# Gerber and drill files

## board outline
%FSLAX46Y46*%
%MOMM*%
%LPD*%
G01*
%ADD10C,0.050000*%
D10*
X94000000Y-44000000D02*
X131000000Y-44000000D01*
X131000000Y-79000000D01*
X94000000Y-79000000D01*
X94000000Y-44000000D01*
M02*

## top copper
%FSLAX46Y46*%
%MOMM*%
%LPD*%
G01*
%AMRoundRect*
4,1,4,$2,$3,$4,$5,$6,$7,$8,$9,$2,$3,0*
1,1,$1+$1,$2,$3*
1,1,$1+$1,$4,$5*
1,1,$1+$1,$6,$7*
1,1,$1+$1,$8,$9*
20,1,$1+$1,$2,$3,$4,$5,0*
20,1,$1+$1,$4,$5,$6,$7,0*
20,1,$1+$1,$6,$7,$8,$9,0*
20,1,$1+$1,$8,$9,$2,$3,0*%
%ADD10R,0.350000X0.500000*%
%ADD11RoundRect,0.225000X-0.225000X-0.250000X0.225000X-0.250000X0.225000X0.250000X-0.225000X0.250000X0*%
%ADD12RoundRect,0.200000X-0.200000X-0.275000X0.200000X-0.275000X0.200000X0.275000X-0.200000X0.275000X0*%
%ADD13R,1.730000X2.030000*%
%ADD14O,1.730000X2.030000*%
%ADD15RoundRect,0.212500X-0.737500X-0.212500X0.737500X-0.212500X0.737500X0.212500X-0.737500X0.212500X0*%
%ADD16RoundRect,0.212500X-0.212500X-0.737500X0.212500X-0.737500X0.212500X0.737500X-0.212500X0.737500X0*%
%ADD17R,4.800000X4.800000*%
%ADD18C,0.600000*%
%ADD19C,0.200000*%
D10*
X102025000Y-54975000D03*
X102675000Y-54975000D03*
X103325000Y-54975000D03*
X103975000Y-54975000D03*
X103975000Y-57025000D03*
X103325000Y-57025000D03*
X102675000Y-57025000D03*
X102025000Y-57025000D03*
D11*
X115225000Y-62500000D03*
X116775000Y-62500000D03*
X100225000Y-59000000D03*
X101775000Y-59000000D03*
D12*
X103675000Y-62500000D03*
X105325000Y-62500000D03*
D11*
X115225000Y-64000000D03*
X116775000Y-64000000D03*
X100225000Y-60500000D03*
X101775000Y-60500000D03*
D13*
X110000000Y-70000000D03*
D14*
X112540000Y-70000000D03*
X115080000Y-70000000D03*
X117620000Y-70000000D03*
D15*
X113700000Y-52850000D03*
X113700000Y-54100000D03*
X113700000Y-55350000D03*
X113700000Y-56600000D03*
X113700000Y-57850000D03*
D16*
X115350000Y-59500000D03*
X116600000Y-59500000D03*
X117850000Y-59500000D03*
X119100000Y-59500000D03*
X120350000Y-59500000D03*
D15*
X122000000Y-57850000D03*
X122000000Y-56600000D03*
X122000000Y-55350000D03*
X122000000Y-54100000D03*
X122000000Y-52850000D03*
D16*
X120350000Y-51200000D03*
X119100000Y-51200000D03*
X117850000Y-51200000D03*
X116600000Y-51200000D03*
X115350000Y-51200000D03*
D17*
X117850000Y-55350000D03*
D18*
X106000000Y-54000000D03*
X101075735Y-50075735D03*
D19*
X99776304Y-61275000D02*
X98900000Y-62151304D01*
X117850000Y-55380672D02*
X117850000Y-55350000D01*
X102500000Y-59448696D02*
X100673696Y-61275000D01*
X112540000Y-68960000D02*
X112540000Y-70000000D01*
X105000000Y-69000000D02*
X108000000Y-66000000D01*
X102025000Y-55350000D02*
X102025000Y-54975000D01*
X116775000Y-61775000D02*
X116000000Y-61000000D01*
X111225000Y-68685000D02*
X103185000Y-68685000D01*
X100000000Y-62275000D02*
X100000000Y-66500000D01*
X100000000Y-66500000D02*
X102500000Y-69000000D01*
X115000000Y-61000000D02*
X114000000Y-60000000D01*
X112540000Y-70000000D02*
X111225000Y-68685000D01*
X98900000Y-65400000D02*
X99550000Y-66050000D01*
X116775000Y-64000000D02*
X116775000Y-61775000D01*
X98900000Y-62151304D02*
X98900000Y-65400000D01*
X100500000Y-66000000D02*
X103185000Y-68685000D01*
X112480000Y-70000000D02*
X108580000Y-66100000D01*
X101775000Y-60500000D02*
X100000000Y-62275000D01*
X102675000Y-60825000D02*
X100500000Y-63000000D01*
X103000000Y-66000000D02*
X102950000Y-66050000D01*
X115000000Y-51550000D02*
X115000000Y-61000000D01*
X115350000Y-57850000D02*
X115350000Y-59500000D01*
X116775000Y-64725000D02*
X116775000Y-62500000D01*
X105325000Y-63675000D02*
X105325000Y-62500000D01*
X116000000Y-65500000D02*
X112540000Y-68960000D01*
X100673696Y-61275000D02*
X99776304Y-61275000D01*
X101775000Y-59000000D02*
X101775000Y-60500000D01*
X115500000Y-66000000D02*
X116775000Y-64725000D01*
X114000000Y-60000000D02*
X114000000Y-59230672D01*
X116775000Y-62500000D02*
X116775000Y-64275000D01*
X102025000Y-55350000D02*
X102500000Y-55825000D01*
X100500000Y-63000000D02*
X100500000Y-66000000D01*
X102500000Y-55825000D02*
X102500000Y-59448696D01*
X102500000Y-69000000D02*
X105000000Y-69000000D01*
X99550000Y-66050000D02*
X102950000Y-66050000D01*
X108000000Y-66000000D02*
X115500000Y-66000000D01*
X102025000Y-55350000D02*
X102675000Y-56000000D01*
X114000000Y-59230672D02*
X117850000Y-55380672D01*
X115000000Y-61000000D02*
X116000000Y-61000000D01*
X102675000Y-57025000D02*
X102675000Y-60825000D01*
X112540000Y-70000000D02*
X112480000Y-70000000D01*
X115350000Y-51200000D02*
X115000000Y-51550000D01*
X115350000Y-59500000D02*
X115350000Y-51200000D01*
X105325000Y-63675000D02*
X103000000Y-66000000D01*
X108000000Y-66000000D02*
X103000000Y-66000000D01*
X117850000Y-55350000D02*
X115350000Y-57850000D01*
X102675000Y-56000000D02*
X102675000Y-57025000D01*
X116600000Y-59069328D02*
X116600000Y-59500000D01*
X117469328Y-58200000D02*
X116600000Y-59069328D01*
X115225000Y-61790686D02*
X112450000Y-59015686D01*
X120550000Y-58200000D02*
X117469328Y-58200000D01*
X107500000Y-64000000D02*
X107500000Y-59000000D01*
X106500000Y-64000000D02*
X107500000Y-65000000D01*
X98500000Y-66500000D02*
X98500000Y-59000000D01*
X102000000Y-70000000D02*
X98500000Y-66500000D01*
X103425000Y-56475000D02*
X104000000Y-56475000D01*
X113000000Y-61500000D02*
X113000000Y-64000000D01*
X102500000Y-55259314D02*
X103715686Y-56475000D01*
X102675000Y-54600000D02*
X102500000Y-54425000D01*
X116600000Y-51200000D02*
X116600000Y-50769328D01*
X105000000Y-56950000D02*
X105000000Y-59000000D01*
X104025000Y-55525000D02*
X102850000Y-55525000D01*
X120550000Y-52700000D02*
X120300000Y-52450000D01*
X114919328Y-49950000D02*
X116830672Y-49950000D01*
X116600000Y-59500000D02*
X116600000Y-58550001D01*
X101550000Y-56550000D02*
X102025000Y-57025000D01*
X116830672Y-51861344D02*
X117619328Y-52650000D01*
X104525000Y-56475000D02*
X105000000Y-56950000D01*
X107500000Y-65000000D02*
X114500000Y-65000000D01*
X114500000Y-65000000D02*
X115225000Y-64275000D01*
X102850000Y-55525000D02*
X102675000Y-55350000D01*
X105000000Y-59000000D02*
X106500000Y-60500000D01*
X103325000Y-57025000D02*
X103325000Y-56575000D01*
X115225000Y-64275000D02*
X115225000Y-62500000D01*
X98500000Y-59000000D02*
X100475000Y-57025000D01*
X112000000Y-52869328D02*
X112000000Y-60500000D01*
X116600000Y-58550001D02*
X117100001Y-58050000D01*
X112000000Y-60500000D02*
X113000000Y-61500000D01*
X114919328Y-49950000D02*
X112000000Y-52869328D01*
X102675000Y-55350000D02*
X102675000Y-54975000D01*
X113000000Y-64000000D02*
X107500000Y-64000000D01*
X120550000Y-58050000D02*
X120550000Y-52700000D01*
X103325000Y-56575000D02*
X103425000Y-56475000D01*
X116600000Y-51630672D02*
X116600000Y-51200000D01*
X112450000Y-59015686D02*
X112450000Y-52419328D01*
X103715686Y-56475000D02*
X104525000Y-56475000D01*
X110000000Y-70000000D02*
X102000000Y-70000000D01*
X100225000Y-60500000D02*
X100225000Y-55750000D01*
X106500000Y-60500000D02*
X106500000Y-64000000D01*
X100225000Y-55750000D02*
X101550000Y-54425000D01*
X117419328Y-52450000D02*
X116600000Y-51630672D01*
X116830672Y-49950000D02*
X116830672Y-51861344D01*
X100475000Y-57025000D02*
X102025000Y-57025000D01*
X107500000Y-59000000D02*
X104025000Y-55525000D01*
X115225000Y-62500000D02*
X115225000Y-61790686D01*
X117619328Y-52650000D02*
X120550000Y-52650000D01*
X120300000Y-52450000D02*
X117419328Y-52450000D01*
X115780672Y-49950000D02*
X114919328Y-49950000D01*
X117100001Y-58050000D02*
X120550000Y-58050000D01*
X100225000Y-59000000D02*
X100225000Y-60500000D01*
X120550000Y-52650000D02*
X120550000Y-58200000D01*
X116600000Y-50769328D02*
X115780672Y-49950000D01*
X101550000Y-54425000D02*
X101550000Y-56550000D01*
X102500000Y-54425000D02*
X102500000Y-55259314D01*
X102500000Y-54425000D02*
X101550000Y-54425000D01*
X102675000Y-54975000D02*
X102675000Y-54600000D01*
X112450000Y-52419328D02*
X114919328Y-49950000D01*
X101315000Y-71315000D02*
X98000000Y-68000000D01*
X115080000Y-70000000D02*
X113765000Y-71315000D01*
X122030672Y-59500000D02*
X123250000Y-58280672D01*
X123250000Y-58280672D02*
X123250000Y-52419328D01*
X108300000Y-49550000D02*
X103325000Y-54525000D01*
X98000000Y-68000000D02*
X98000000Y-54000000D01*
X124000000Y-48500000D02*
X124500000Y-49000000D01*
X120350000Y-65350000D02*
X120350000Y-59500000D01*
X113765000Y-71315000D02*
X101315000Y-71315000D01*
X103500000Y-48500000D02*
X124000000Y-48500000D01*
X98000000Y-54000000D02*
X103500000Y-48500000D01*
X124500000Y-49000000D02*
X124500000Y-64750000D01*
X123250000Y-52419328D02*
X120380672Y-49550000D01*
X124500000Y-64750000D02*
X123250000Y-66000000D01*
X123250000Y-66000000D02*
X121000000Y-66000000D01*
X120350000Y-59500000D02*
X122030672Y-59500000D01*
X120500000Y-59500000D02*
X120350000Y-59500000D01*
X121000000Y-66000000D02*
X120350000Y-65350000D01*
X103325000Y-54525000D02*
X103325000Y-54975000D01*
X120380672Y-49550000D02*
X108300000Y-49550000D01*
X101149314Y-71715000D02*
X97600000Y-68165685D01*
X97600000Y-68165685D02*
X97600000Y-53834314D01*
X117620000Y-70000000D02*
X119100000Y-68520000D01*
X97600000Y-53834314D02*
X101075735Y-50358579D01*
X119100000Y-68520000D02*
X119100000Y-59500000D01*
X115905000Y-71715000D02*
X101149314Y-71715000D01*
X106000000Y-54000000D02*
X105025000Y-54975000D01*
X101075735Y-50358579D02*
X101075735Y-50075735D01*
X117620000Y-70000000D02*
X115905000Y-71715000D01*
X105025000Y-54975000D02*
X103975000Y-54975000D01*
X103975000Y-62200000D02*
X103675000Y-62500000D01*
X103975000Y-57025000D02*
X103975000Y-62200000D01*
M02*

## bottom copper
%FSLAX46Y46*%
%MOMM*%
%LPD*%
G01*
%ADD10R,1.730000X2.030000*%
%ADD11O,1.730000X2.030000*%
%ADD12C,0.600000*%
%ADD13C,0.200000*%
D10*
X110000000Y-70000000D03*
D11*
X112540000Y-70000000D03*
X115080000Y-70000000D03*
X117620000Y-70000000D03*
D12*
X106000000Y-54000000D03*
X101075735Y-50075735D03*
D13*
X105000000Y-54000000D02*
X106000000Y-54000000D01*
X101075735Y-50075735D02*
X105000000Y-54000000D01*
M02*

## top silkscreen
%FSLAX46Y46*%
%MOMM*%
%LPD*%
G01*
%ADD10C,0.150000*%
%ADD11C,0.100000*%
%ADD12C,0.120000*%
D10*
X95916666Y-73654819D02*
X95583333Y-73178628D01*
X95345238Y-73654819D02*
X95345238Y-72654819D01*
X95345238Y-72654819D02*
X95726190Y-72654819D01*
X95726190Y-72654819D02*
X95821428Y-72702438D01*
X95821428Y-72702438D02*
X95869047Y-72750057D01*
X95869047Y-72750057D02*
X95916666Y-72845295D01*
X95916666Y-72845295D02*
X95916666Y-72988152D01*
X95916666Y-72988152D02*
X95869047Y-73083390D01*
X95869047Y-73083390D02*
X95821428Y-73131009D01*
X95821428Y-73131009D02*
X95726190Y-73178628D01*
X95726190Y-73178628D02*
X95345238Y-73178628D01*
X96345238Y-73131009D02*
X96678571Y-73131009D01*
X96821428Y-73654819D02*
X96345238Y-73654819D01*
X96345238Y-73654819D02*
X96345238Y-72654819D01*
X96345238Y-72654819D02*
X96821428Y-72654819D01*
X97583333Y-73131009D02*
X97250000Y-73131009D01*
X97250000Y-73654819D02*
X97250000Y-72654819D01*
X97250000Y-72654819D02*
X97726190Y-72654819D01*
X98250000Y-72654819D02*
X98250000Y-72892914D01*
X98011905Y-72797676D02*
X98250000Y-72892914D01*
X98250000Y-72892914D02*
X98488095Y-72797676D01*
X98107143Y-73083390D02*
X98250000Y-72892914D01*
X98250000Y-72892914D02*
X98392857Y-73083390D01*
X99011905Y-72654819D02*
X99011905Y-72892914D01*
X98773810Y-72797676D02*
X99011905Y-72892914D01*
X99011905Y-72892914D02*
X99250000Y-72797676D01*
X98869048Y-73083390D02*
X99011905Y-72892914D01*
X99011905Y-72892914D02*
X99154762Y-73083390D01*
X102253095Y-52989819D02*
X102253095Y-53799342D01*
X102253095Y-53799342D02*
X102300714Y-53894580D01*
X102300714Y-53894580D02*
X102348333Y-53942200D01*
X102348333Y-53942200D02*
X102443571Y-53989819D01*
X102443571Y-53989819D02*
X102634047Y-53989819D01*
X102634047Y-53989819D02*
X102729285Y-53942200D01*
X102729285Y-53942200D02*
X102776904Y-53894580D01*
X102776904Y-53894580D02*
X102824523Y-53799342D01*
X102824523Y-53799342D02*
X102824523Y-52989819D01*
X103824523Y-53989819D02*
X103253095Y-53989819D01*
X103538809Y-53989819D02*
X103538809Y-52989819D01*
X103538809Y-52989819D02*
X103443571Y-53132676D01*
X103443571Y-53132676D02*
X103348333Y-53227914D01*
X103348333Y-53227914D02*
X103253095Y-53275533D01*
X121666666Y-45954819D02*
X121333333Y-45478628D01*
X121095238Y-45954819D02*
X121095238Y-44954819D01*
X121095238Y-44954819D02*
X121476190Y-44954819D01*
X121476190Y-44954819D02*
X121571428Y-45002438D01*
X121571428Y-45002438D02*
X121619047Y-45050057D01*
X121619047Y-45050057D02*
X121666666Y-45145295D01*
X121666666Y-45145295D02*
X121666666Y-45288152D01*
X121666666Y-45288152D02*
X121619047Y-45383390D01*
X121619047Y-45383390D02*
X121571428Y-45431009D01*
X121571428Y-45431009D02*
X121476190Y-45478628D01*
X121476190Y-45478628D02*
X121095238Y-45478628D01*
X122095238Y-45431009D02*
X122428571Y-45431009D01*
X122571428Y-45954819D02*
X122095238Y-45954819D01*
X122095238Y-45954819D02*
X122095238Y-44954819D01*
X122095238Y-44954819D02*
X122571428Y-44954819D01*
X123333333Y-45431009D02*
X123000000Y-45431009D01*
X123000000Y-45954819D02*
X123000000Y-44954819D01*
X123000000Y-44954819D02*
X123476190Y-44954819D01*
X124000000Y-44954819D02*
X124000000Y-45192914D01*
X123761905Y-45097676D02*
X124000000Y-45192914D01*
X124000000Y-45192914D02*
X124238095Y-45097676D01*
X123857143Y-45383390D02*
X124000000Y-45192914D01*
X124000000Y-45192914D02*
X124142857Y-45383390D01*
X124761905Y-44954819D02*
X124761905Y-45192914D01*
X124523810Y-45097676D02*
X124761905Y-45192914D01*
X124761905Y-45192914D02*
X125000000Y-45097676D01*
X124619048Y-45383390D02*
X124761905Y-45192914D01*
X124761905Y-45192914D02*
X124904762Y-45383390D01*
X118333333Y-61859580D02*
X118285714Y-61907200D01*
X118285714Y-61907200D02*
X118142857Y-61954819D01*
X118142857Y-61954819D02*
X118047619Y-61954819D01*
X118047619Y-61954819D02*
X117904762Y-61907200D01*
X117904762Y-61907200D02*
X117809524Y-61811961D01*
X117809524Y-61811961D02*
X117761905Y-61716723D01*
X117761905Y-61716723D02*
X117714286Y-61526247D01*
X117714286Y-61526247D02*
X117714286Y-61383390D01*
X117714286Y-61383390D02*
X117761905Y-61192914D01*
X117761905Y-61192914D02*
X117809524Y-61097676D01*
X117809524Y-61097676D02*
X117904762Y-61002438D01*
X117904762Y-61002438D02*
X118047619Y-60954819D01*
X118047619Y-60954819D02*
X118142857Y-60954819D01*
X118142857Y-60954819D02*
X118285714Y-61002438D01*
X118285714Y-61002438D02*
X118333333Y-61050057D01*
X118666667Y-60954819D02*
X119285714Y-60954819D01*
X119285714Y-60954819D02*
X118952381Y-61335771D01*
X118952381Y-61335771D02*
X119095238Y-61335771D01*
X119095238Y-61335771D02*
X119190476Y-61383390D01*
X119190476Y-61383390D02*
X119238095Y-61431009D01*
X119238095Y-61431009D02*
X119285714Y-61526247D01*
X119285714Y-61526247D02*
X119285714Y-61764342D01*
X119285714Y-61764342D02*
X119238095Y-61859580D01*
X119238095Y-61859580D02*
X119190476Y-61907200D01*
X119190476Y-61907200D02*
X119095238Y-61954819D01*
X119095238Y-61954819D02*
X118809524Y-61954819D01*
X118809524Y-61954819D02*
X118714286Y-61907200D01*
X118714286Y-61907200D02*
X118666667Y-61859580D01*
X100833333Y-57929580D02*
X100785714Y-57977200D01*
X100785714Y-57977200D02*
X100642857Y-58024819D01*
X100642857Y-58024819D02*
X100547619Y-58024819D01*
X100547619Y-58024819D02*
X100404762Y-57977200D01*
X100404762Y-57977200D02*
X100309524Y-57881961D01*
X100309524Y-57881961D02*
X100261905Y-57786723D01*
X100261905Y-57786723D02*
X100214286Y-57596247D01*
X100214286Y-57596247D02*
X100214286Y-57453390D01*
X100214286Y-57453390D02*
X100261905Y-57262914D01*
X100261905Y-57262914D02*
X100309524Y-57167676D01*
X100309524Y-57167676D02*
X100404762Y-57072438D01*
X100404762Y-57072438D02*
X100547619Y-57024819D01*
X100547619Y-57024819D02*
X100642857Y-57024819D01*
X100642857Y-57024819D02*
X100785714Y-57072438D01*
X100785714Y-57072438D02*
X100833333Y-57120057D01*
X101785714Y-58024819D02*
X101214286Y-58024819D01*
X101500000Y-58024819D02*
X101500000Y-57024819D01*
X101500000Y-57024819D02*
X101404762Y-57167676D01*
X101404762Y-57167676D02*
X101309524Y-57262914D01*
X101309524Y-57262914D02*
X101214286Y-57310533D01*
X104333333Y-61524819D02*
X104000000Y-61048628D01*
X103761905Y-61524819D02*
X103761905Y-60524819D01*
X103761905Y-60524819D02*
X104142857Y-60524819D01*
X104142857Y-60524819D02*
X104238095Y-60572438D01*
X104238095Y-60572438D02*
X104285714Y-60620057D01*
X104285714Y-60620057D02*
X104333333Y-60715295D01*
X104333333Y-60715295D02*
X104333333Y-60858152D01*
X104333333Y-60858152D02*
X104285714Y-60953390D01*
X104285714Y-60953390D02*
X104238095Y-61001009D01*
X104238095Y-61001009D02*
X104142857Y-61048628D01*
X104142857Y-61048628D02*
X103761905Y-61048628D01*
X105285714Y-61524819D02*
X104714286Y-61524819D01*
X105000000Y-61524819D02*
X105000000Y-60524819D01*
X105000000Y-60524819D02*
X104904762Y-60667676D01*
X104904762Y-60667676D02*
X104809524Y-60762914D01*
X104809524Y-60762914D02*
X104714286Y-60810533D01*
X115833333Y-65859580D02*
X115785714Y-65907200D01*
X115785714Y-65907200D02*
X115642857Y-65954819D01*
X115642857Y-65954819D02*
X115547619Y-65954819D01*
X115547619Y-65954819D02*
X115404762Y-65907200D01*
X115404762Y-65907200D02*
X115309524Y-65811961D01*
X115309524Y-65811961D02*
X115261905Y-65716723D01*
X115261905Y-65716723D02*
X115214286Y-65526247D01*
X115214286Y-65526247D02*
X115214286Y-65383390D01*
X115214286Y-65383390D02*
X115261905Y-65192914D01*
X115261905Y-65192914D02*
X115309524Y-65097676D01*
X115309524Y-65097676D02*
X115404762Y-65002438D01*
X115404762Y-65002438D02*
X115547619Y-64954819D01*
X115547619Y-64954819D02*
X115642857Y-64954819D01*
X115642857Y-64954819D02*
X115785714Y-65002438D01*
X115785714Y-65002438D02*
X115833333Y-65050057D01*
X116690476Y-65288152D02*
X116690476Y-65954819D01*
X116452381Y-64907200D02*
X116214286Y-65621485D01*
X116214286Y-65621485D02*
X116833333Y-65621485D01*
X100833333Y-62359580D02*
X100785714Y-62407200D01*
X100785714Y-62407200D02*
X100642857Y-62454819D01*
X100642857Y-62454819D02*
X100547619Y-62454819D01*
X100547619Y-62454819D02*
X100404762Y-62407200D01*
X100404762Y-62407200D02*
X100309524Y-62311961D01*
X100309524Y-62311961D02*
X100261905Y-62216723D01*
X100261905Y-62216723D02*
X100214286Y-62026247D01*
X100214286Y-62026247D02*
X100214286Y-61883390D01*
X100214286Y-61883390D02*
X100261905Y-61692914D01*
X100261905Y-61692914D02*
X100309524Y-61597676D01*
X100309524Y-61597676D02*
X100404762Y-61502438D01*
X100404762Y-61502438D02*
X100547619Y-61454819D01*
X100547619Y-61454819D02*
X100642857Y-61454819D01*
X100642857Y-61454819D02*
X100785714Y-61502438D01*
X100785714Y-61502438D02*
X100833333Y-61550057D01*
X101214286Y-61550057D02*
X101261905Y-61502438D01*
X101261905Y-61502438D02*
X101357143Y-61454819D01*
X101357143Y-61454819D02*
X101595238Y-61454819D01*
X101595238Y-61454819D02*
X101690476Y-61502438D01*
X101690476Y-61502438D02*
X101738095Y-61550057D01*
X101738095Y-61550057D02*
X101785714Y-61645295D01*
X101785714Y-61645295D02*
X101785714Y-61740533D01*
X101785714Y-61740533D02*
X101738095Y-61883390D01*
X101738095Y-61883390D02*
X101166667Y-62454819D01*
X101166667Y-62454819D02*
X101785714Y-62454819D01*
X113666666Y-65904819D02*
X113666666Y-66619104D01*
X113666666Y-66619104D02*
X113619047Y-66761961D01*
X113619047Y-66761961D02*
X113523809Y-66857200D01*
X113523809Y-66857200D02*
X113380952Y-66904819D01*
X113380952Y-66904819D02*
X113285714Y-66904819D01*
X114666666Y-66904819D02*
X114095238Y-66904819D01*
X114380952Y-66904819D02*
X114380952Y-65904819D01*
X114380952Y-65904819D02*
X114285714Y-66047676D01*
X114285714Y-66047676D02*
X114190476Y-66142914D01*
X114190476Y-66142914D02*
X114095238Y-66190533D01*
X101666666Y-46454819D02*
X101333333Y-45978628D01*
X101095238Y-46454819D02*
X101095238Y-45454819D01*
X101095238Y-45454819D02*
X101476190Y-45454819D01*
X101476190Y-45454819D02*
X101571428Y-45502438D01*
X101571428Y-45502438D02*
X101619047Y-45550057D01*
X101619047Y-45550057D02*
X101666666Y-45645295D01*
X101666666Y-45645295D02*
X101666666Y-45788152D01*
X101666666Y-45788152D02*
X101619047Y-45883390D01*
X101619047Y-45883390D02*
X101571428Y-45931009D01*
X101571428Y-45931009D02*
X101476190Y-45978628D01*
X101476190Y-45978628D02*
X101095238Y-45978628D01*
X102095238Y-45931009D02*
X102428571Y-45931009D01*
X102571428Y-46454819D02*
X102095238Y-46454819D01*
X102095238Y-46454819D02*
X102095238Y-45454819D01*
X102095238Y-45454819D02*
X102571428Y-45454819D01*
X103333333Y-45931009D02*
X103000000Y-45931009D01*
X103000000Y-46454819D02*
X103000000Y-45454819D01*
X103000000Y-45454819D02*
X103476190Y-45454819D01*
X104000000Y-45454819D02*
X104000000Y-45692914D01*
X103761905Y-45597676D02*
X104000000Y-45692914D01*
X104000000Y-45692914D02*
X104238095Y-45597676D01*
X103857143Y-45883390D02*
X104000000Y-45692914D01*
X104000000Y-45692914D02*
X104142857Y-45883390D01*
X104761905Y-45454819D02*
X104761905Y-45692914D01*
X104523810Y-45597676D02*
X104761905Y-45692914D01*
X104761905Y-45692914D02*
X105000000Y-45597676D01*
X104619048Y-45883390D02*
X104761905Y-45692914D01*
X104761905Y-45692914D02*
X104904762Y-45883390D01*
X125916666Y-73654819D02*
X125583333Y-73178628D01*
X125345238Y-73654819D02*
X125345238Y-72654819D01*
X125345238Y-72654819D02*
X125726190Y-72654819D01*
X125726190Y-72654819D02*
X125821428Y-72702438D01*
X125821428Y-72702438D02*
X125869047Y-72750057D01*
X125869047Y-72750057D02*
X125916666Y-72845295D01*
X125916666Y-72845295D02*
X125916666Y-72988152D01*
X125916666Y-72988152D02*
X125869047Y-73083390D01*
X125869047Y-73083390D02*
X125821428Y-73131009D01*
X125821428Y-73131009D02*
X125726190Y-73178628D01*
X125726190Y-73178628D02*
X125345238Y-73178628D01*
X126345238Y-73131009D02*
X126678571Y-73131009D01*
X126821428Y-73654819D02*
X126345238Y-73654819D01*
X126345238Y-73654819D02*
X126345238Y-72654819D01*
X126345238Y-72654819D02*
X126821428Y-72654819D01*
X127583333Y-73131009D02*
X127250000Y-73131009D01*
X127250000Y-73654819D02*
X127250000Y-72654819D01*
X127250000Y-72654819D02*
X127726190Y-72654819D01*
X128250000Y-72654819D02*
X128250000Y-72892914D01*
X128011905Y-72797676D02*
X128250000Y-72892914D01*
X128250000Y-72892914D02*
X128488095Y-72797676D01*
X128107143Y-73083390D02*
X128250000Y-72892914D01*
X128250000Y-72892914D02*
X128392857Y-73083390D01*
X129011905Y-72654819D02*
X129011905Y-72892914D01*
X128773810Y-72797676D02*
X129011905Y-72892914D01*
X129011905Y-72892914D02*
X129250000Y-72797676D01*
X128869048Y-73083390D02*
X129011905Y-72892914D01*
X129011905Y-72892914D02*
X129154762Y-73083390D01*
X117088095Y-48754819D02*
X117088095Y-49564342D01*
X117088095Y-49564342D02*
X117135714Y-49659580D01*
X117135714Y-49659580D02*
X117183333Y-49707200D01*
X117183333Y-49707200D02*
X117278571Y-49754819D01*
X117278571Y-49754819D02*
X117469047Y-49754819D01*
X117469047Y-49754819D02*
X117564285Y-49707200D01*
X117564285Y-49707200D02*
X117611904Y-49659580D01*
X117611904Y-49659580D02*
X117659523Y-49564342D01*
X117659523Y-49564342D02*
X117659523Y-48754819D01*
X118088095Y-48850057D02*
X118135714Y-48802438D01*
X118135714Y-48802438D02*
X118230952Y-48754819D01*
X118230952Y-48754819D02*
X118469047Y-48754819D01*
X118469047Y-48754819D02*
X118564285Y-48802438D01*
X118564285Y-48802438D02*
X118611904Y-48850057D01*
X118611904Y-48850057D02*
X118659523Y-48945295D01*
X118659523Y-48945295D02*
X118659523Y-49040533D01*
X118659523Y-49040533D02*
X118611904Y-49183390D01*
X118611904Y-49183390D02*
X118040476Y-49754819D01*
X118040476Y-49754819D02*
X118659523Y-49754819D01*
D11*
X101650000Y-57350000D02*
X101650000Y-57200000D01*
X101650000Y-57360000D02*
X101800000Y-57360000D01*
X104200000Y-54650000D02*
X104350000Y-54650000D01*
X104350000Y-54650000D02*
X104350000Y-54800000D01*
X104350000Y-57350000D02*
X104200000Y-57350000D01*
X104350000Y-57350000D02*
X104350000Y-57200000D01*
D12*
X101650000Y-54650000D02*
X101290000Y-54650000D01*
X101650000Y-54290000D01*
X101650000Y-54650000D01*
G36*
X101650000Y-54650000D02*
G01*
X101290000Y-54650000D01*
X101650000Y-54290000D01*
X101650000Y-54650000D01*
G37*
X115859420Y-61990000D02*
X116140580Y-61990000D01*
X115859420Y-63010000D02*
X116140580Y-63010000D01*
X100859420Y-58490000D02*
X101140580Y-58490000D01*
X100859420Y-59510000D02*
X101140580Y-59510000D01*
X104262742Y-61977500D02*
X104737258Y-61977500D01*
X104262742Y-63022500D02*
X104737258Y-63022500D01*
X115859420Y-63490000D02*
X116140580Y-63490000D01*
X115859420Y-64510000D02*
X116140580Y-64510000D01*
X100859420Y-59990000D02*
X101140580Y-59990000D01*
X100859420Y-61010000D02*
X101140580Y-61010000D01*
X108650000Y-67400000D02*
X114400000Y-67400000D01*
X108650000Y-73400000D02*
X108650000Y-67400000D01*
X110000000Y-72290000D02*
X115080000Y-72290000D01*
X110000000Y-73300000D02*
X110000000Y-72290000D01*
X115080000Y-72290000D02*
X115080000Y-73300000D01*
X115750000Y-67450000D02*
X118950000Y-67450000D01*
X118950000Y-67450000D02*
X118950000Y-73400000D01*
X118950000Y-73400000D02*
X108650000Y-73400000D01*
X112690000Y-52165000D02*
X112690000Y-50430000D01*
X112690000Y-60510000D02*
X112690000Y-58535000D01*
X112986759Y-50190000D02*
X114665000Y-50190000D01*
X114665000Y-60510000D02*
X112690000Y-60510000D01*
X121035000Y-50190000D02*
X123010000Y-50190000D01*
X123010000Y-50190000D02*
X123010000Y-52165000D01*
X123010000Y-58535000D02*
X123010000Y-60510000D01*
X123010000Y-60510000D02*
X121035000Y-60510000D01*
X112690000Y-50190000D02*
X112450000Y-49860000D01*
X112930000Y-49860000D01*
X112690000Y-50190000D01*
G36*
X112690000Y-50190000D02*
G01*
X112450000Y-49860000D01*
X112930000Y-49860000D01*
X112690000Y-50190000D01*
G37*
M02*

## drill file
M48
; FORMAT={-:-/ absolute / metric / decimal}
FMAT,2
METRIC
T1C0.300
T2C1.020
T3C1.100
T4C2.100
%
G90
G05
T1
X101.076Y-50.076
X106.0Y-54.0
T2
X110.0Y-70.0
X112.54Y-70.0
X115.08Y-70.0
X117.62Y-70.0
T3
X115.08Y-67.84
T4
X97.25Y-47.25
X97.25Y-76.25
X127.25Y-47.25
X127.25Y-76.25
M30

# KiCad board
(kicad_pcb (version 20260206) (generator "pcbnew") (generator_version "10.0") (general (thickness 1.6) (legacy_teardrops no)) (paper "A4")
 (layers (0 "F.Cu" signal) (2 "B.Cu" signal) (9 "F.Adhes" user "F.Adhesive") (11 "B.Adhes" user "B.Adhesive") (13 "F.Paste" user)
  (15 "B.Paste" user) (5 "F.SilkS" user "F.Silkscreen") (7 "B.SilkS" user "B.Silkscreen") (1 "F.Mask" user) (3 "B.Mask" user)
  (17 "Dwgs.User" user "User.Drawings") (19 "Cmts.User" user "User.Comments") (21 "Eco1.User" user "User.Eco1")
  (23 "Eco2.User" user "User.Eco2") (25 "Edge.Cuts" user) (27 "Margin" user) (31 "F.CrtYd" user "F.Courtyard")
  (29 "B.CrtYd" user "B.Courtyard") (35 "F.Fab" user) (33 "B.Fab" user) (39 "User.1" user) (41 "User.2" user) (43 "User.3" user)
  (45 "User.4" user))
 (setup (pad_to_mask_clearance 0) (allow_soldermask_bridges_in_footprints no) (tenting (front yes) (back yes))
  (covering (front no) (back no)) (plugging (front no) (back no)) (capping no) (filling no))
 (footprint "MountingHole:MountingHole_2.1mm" (layer "F.Cu") (at 97.25 76.25)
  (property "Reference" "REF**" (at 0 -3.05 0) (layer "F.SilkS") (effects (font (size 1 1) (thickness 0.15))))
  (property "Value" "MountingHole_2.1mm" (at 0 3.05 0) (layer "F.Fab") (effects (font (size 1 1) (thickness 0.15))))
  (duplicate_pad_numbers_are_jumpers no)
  (pad "" np_thru_hole circle (at 0 0) (size 2.1 2.1) (drill 2.1) (layers "*.Cu" "*.Mask")))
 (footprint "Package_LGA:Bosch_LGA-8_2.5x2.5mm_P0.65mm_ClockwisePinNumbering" (layer "F.Cu") (at 103 56)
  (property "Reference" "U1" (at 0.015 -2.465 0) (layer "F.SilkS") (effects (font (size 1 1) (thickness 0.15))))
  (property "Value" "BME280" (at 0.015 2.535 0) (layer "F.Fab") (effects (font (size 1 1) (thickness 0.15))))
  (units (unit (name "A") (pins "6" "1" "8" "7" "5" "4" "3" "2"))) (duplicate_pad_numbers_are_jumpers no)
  (fp_line (start -1.35 1.35) (end -1.35 1.2) (stroke (width 0.1) (type solid)) (layer "F.SilkS"))
  (fp_line (start -1.35 1.36) (end -1.2 1.36) (stroke (width 0.1) (type solid)) (layer "F.SilkS"))
  (fp_line (start 1.2 -1.35) (end 1.35 -1.35) (stroke (width 0.1) (type solid)) (layer "F.SilkS"))
  (fp_line (start 1.35 -1.35) (end 1.35 -1.2) (stroke (width 0.1) (type solid)) (layer "F.SilkS"))
  (fp_line (start 1.35 1.35) (end 1.2 1.35) (stroke (width 0.1) (type solid)) (layer "F.SilkS"))
  (fp_line (start 1.35 1.35) (end 1.35 1.2) (stroke (width 0.1) (type solid)) (layer "F.SilkS"))
  (fp_poly
   (pts (xy -1.35 -1.35) (xy -1.71 -1.35) (xy -1.35 -1.71) (xy -1.35 -1.35)) (stroke (width 0.12) (type solid)) (fill yes) (layer "F.SilkS"))
  (pad "1" smd rect (at -0.975 -1.025 90) (size 0.5 0.35) (layers "F.Cu" "F.Mask" "F.Paste") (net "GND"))
  (pad "2" smd rect (at -0.325 -1.025 90) (size 0.5 0.35) (layers "F.Cu" "F.Mask" "F.Paste") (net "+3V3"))
  (pad "3" smd rect (at 0.325 -1.025 90) (size 0.5 0.35) (layers "F.Cu" "F.Mask" "F.Paste") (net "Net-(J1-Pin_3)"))
  (pad "4" smd rect (at 0.975 -1.025 90) (size 0.5 0.35) (layers "F.Cu" "F.Mask" "F.Paste") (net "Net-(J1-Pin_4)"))
  (pad "5" smd rect (at 0.975 1.025 90) (size 0.5 0.35) (layers "F.Cu" "F.Mask" "F.Paste") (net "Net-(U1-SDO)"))
  (pad "6" smd rect (at 0.325 1.025 90) (size 0.5 0.35) (layers "F.Cu" "F.Mask" "F.Paste") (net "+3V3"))
  (pad "7" smd rect (at -0.325 1.025 90) (size 0.5 0.35) (layers "F.Cu" "F.Mask" "F.Paste") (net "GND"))
  (pad "8" smd rect (at -0.975 1.025 90) (size 0.5 0.35) (layers "F.Cu" "F.Mask" "F.Paste") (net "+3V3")))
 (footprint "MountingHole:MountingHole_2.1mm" (layer "F.Cu") (at 127.25 47.25)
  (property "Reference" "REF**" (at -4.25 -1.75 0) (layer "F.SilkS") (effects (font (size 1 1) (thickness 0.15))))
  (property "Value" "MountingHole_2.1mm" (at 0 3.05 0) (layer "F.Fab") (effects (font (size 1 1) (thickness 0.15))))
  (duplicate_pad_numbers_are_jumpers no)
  (pad "" np_thru_hole circle (at 0 0) (size 2.1 2.1) (drill 2.1) (layers "*.Cu" "*.Mask")))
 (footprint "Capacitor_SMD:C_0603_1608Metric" (layer "F.Cu") (at 116 62.5)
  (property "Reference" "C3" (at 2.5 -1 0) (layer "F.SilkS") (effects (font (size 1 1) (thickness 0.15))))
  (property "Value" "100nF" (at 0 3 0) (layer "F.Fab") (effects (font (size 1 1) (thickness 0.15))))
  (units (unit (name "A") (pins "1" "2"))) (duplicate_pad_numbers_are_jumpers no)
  (fp_line (start -0.14058 -0.51) (end 0.14058 -0.51) (stroke (width 0.12) (type solid)) (layer "F.SilkS"))
  (fp_line (start -0.14058 0.51) (end 0.14058 0.51) (stroke (width 0.12) (type solid)) (layer "F.SilkS"))
  (pad "1" smd roundrect (at -0.775 0) (size 0.9 0.95) (layers "F.Cu" "F.Mask" "F.Paste") (roundrect_rratio 0.25) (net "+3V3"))
  (pad "2" smd roundrect (at 0.775 0) (size 0.9 0.95) (layers "F.Cu" "F.Mask" "F.Paste") (roundrect_rratio 0.25) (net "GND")))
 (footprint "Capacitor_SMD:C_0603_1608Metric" (layer "F.Cu") (at 101 59)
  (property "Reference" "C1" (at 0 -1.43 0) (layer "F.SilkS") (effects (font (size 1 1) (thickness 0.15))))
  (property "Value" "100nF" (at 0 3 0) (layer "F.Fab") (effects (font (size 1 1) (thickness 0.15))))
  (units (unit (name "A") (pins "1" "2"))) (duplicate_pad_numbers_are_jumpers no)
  (fp_line (start -0.14058 -0.51) (end 0.14058 -0.51) (stroke (width 0.12) (type solid)) (layer "F.SilkS"))
  (fp_line (start -0.14058 0.51) (end 0.14058 0.51) (stroke (width 0.12) (type solid)) (layer "F.SilkS"))
  (pad "1" smd roundrect (at -0.775 0) (size 0.9 0.95) (layers "F.Cu" "F.Mask" "F.Paste") (roundrect_rratio 0.25) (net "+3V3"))
  (pad "2" smd roundrect (at 0.775 0) (size 0.9 0.95) (layers "F.Cu" "F.Mask" "F.Paste") (roundrect_rratio 0.25) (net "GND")))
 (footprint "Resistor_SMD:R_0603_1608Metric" (layer "F.Cu") (at 104.5 62.5)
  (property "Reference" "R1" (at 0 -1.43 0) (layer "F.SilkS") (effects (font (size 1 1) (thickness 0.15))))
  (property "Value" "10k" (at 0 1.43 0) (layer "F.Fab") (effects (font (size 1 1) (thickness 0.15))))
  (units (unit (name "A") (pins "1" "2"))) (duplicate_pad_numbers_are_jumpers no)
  (fp_line (start -0.237258 -0.5225) (end 0.237258 -0.5225) (stroke (width 0.12) (type solid)) (layer "F.SilkS"))
  (fp_line (start -0.237258 0.5225) (end 0.237258 0.5225) (stroke (width 0.12) (type solid)) (layer "F.SilkS"))
  (pad "1" smd roundrect (at -0.825 0) (size 0.8 0.95) (layers "F.Cu" "F.Mask" "F.Paste") (roundrect_rratio 0.25) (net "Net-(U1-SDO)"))
  (pad "2" smd roundrect (at 0.825 0) (size 0.8 0.95) (layers "F.Cu" "F.Mask" "F.Paste") (roundrect_rratio 0.25) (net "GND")))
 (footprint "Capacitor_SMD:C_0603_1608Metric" (layer "F.Cu") (at 116 64)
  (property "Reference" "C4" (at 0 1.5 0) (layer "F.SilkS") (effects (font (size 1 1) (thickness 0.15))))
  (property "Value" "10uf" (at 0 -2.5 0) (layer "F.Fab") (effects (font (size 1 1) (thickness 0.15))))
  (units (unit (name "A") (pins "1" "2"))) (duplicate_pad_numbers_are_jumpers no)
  (fp_line (start -0.14058 -0.51) (end 0.14058 -0.51) (stroke (width 0.12) (type solid)) (layer "F.SilkS"))
  (fp_line (start -0.14058 0.51) (end 0.14058 0.51) (stroke (width 0.12) (type solid)) (layer "F.SilkS"))
  (pad "1" smd roundrect (at -0.775 0) (size 0.9 0.95) (layers "F.Cu" "F.Mask" "F.Paste") (roundrect_rratio 0.25) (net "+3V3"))
  (pad "2" smd roundrect (at 0.775 0) (size 0.9 0.95) (layers "F.Cu" "F.Mask" "F.Paste") (roundrect_rratio 0.25) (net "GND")))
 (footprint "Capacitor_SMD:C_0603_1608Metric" (layer "F.Cu") (at 101 60.5)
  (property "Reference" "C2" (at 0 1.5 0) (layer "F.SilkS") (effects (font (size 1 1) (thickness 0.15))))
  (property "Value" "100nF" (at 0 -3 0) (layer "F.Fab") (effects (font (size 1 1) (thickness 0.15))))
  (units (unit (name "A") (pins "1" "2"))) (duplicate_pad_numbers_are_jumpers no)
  (fp_line (start -0.14058 -0.51) (end 0.14058 -0.51) (stroke (width 0.12) (type solid)) (layer "F.SilkS"))
  (fp_line (start -0.14058 0.51) (end 0.14058 0.51) (stroke (width 0.12) (type solid)) (layer "F.SilkS"))
  (pad "1" smd roundrect (at -0.775 0) (size 0.9 0.95) (layers "F.Cu" "F.Mask" "F.Paste") (roundrect_rratio 0.25) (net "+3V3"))
  (pad "2" smd roundrect (at 0.775 0) (size 0.9 0.95) (layers "F.Cu" "F.Mask" "F.Paste") (roundrect_rratio 0.25) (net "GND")))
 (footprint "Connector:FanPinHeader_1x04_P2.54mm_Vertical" (layer "F.Cu") (at 110 70)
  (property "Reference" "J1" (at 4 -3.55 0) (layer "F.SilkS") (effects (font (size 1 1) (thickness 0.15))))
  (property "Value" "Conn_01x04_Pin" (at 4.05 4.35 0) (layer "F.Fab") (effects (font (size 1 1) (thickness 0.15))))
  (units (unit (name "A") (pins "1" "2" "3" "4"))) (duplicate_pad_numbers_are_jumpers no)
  (fp_line (start -1.35 -2.6) (end 4.4 -2.6) (stroke (width 0.12) (type solid)) (layer "F.SilkS"))
  (fp_line (start -1.35 3.4) (end -1.35 -2.6) (stroke (width 0.12) (type solid)) (layer "F.SilkS"))
  (fp_line (start 0 2.29) (end 5.08 2.29) (stroke (width 0.12) (type solid)) (layer "F.SilkS"))
  (fp_line (start 0 3.3) (end 0 2.29) (stroke (width 0.12) (type solid)) (layer "F.SilkS"))
  (fp_line (start 5.08 2.29) (end 5.08 3.3) (stroke (width 0.12) (type solid)) (layer "F.SilkS"))
  (fp_line (start 5.75 -2.55) (end 8.95 -2.55) (stroke (width 0.12) (type solid)) (layer "F.SilkS"))
  (fp_line (start 8.95 -2.55) (end 8.95 3.4) (stroke (width 0.12) (type solid)) (layer "F.SilkS"))
  (fp_line (start 8.95 3.4) (end -1.35 3.4) (stroke (width 0.12) (type solid)) (layer "F.SilkS"))
  (pad "" np_thru_hole circle (at 5.08 -2.16 90) (size 1.1 1.1) (drill 1.1) (layers "*.Cu" "*.Mask"))
  (pad "1" thru_hole rect (at 0 0 90) (size 2.03 1.73) (drill 1.02) (layers "*.Cu" "*.Mask") (remove_unused_layers no) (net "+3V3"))
  (pad "2" thru_hole oval (at 2.54 0 90) (size 2.03 1.73) (drill 1.02) (layers "*.Cu" "*.Mask") (remove_unused_layers no) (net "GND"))
  (pad "3" thru_hole oval (at 5.08 0 90) (size 2.03 1.73) (drill 1.02) (layers "*.Cu" "*.Mask") (remove_unused_layers no)
   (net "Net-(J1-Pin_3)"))
  (pad "4" thru_hole oval (at 7.62 0 90) (size 2.03 1.73) (drill 1.02) (layers "*.Cu" "*.Mask") (remove_unused_layers no)
   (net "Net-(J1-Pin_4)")))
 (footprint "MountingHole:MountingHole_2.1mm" (layer "F.Cu") (at 97.25 47.25)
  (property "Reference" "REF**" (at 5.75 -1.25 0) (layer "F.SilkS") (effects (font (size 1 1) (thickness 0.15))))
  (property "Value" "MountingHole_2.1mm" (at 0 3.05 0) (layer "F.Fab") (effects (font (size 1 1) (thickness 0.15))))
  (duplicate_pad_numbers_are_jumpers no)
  (pad "" np_thru_hole circle (at 0 0) (size 2.1 2.1) (drill 2.1) (layers "*.Cu" "*.Mask")))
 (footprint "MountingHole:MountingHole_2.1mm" (layer "F.Cu") (at 127.25 76.25)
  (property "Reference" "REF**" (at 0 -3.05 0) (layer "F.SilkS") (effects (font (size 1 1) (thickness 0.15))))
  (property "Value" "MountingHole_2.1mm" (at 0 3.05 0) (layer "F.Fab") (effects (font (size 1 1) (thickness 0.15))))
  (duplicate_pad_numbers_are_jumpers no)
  (pad "" np_thru_hole circle (at 0 0) (size 2.1 2.1) (drill 2.1) (layers "*.Cu" "*.Mask")))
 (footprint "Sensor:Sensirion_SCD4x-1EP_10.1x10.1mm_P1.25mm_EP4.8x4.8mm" (layer "F.Cu") (at 117.85 55.35)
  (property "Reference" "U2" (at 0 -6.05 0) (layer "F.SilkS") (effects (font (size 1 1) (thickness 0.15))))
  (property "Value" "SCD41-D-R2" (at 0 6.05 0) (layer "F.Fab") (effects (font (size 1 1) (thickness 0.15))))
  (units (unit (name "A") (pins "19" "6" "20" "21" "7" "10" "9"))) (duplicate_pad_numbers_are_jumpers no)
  (fp_line (start -5.16 -3.185) (end -5.16 -4.92) (stroke (width 0.12) (type solid)) (layer "F.SilkS"))
  (fp_line (start -5.16 5.16) (end -5.16 3.185) (stroke (width 0.12) (type solid)) (layer "F.SilkS"))
  (fp_line (start -4.863241 -5.16) (end -3.185 -5.16) (stroke (width 0.12) (type solid)) (layer "F.SilkS"))
  (fp_line (start -3.185 5.16) (end -5.16 5.16) (stroke (width 0.12) (type solid)) (layer "F.SilkS"))
  (fp_line (start 3.185 -5.16) (end 5.16 -5.16) (stroke (width 0.12) (type solid)) (layer "F.SilkS"))
  (fp_line (start 5.16 -5.16) (end 5.16 -3.185) (stroke (width 0.12) (type solid)) (layer "F.SilkS"))
  (fp_line (start 5.16 3.185) (end 5.16 5.16) (stroke (width 0.12) (type solid)) (layer "F.SilkS"))
  (fp_line (start 5.16 5.16) (end 3.185 5.16) (stroke (width 0.12) (type solid)) (layer "F.SilkS"))
  (fp_poly (pts (xy -5.16 -5.16) (xy -5.4 -5.49) (xy -4.92 -5.49)) (stroke (width 0.12) (type solid)) (fill yes) (layer "F.SilkS"))
  (pad "" smd roundrect (at -1.2 -1.2) (size 1.93 1.93) (layers "F.Paste") (roundrect_rratio 0.129534))
  (pad "" smd roundrect (at -1.2 1.2) (size 1.93 1.93) (layers "F.Paste") (roundrect_rratio 0.129534))
  (pad "" smd roundrect (at 1.2 -1.2) (size 1.93 1.93) (layers "F.Paste") (roundrect_rratio 0.129534))
  (pad "" smd roundrect (at 1.2 1.2) (size 1.93 1.93) (layers "F.Paste") (roundrect_rratio 0.129534))
  (pad "1" smd roundrect (at -4.15 -2.5) (size 1.9 0.85) (layers "F.Cu" "F.Mask" "F.Paste") (roundrect_rratio 0.25))
  (pad "2" smd roundrect (at -4.15 -1.25) (size 1.9 0.85) (layers "F.Cu" "F.Mask" "F.Paste") (roundrect_rratio 0.25))
  (pad "3" smd roundrect (at -4.15 0) (size 1.9 0.85) (layers "F.Cu" "F.Mask" "F.Paste") (roundrect_rratio 0.25))
  (pad "4" smd roundrect (at -4.15 1.25) (size 1.9 0.85) (layers "F.Cu" "F.Mask" "F.Paste") (roundrect_rratio 0.25))
  (pad "5" smd roundrect (at -4.15 2.5) (size 1.9 0.85) (layers "F.Cu" "F.Mask" "F.Paste") (roundrect_rratio 0.25))
  (pad "6" smd roundrect (at -2.5 4.15) (size 0.85 1.9) (layers "F.Cu" "F.Mask" "F.Paste") (roundrect_rratio 0.25) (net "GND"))
  (pad "7" smd roundrect (at -1.25 4.15) (size 0.85 1.9) (layers "F.Cu" "F.Mask" "F.Paste") (roundrect_rratio 0.25) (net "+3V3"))
  (pad "8" smd roundrect (at 0 4.15) (size 0.85 1.9) (layers "F.Cu" "F.Mask" "F.Paste") (roundrect_rratio 0.25))
  (pad "9" smd roundrect (at 1.25 4.15) (size 0.85 1.9) (layers "F.Cu" "F.Mask" "F.Paste") (roundrect_rratio 0.25) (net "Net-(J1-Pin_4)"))
  (pad "10" smd roundrect (at 2.5 4.15) (size 0.85 1.9) (layers "F.Cu" "F.Mask" "F.Paste") (roundrect_rratio 0.25) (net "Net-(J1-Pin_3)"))
  (pad "11" smd roundrect (at 4.15 2.5) (size 1.9 0.85) (layers "F.Cu" "F.Mask" "F.Paste") (roundrect_rratio 0.25))
  (pad "12" smd roundrect (at 4.15 1.25) (size 1.9 0.85) (layers "F.Cu" "F.Mask" "F.Paste") (roundrect_rratio 0.25))
  (pad "13" smd roundrect (at 4.15 0) (size 1.9 0.85) (layers "F.Cu" "F.Mask" "F.Paste") (roundrect_rratio 0.25))
  (pad "14" smd roundrect (at 4.15 -1.25) (size 1.9 0.85) (layers "F.Cu" "F.Mask" "F.Paste") (roundrect_rratio 0.25))
  (pad "15" smd roundrect (at 4.15 -2.5) (size 1.9 0.85) (layers "F.Cu" "F.Mask" "F.Paste") (roundrect_rratio 0.25))
  (pad "16" smd roundrect (at 2.5 -4.15) (size 0.85 1.9) (layers "F.Cu" "F.Mask" "F.Paste") (roundrect_rratio 0.25))
  (pad "17" smd roundrect (at 1.25 -4.15) (size 0.85 1.9) (layers "F.Cu" "F.Mask" "F.Paste") (roundrect_rratio 0.25))
  (pad "18" smd roundrect (at 0 -4.15) (size 0.85 1.9) (layers "F.Cu" "F.Mask" "F.Paste") (roundrect_rratio 0.25))
  (pad "19" smd roundrect (at -1.25 -4.15) (size 0.85 1.9) (layers "F.Cu" "F.Mask" "F.Paste") (roundrect_rratio 0.25) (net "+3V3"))
  (pad "20" smd roundrect (at -2.5 -4.15) (size 0.85 1.9) (layers "F.Cu" "F.Mask" "F.Paste") (roundrect_rratio 0.25) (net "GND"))
  (pad "21" smd rect (at 0 0) (size 4.8 4.8) (layers "F.Cu" "F.Mask") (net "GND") (zone_connect 2)))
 (gr_rect (start 94 44) (end 131 79) (stroke (width 0.05) (type default)) (fill no) (layer "Edge.Cuts"))
 (segment (start 99.776304 61.275) (end 98.9 62.151304) (width 0.2) (layer "F.Cu") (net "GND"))
 (segment (start 117.85 55.380672) (end 117.85 55.35) (width 0.2) (layer "F.Cu") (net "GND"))
 (segment (start 102.5 59.448696) (end 100.673696 61.275) (width 0.2) (layer "F.Cu") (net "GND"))
 (segment (start 112.54 68.96) (end 112.54 70) (width 0.2) (layer "F.Cu") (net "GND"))
 (segment (start 105 69) (end 108 66) (width 0.2) (layer "F.Cu") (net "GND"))
 (segment (start 102.025 55.35) (end 102.025 54.975) (width 0.2) (layer "F.Cu") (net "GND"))
 (segment (start 116.775 61.775) (end 116 61) (width 0.2) (layer "F.Cu") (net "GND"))
 (segment (start 111.225 68.685) (end 103.185 68.685) (width 0.2) (layer "F.Cu") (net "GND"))
 (segment (start 100 62.275) (end 100 66.5) (width 0.2) (layer "F.Cu") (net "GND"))
 (segment (start 100 66.5) (end 102.5 69) (width 0.2) (layer "F.Cu") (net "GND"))
 (segment (start 115 61) (end 114 60) (width 0.2) (layer "F.Cu") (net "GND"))
 (segment (start 112.54 70) (end 111.225 68.685) (width 0.2) (layer "F.Cu") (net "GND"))
 (segment (start 98.9 65.4) (end 99.55 66.05) (width 0.2) (layer "F.Cu") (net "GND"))
 (segment (start 116.775 64) (end 116.775 61.775) (width 0.2) (layer "F.Cu") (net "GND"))
 (segment (start 98.9 62.151304) (end 98.9 65.4) (width 0.2) (layer "F.Cu") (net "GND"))
 (segment (start 100.5 66) (end 103.185 68.685) (width 0.2) (layer "F.Cu") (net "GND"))
 (segment (start 112.48 70) (end 108.58 66.1) (width 0.2) (layer "F.Cu") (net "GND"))
 (segment (start 101.775 60.5) (end 100 62.275) (width 0.2) (layer "F.Cu") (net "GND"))
 (segment (start 102.675 60.825) (end 100.5 63) (width 0.2) (layer "F.Cu") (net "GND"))
 (segment (start 103 66) (end 102.95 66.05) (width 0.2) (layer "F.Cu") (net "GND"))
 (segment (start 115 51.55) (end 115 61) (width 0.2) (layer "F.Cu") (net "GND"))
 (segment (start 115.35 57.85) (end 115.35 59.5) (width 0.2) (layer "F.Cu") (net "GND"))
 (segment (start 116.775 64.725) (end 116.775 62.5) (width 0.2) (layer "F.Cu") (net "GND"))
 (segment (start 105.325 63.675) (end 105.325 62.5) (width 0.2) (layer "F.Cu") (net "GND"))
 (segment (start 116 65.5) (end 112.54 68.96) (width 0.2) (layer "F.Cu") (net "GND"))
 (segment (start 100.673696 61.275) (end 99.776304 61.275) (width 0.2) (layer "F.Cu") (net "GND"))
 (segment (start 101.775 59) (end 101.775 60.5) (width 0.2) (layer "F.Cu") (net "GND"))
 (segment (start 115.5 66) (end 116.775 64.725) (width 0.2) (layer "F.Cu") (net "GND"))
 (segment (start 114 60) (end 114 59.230672) (width 0.2) (layer "F.Cu") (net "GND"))
 (segment (start 116.775 62.5) (end 116.775 64.275) (width 0.2) (layer "F.Cu") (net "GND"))
 (segment (start 102.025 55.35) (end 102.5 55.825) (width 0.2) (layer "F.Cu") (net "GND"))
 (segment (start 100.5 63) (end 100.5 66) (width 0.2) (layer "F.Cu") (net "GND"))
 (segment (start 102.5 55.825) (end 102.5 59.448696) (width 0.2) (layer "F.Cu") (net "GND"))
 (segment (start 102.5 69) (end 105 69) (width 0.2) (layer "F.Cu") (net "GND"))
 (segment (start 99.55 66.05) (end 102.95 66.05) (width 0.2) (layer "F.Cu") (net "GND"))
 (segment (start 108 66) (end 115.5 66) (width 0.2) (layer "F.Cu") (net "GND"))
 (segment (start 102.025 55.35) (end 102.675 56) (width 0.2) (layer "F.Cu") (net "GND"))
 (segment (start 114 59.230672) (end 117.85 55.380672) (width 0.2) (layer "F.Cu") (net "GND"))
 (segment (start 115 61) (end 116 61) (width 0.2) (layer "F.Cu") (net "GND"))
 (segment (start 102.675 57.025) (end 102.675 60.825) (width 0.2) (layer "F.Cu") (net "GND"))
 (segment (start 112.54 70) (end 112.48 70) (width 0.2) (layer "F.Cu") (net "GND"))
 (segment (start 115.35 51.2) (end 115 51.55) (width 0.2) (layer "F.Cu") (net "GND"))
 (segment (start 115.35 59.5) (end 115.35 51.2) (width 0.2) (layer "F.Cu") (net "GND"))
 (segment (start 105.325 63.675) (end 103 66) (width 0.2) (layer "F.Cu") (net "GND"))
 (segment (start 108 66) (end 103 66) (width 0.2) (layer "F.Cu") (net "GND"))
 (segment (start 117.85 55.35) (end 115.35 57.85) (width 0.2) (layer "F.Cu") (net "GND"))
 (segment (start 102.675 56) (end 102.675 57.025) (width 0.2) (layer "F.Cu") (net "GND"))
 (segment (start 116.6 59.069328) (end 116.6 59.5) (width 0.2) (layer "F.Cu") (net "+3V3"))
 (segment (start 117.469328 58.2) (end 116.6 59.069328) (width 0.2) (layer "F.Cu") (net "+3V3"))
 (segment (start 115.225 61.790686) (end 112.45 59.015686) (width 0.2) (layer "F.Cu") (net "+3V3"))
 (segment (start 120.55 58.2) (end 117.469328 58.2) (width 0.2) (layer "F.Cu") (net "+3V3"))
 (segment (start 107.5 64) (end 107.5 59) (width 0.2) (layer "F.Cu") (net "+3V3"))
 (segment (start 106.5 64) (end 107.5 65) (width 0.2) (layer "F.Cu") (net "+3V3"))
 (segment (start 98.5 66.5) (end 98.5 59) (width 0.2) (layer "F.Cu") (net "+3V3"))
 (segment (start 102 70) (end 98.5 66.5) (width 0.2) (layer "F.Cu") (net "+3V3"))
 (segment (start 103.425 56.475) (end 104 56.475) (width 0.2) (layer "F.Cu") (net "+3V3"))
 (segment (start 113 61.5) (end 113 64) (width 0.2) (layer "F.Cu") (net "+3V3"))
 (segment (start 102.5 55.259314) (end 103.715686 56.475) (width 0.2) (layer "F.Cu") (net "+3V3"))
 (segment (start 102.675 54.6) (end 102.5 54.425) (width 0.2) (layer "F.Cu") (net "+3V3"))
 (segment (start 116.6 51.2) (end 116.6 50.769328) (width 0.2) (layer "F.Cu") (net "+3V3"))
 (segment (start 105 56.95) (end 105 59) (width 0.2) (layer "F.Cu") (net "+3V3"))
 (segment (start 104.025 55.525) (end 102.85 55.525) (width 0.2) (layer "F.Cu") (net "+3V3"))
 (segment (start 120.55 52.7) (end 120.3 52.45) (width 0.2) (layer "F.Cu") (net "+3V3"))
 (segment (start 114.919328 49.95) (end 116.830672 49.95) (width 0.2) (layer "F.Cu") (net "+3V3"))
 (segment (start 116.6 59.5) (end 116.6 58.550001) (width 0.2) (layer "F.Cu") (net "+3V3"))
 (segment (start 101.55 56.55) (end 102.025 57.025) (width 0.2) (layer "F.Cu") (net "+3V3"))
 (segment (start 116.830672 51.861344) (end 117.619328 52.65) (width 0.2) (layer "F.Cu") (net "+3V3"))
 (segment (start 104.525 56.475) (end 105 56.95) (width 0.2) (layer "F.Cu") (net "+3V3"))
 (segment (start 107.5 65) (end 114.5 65) (width 0.2) (layer "F.Cu") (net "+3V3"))
 (segment (start 114.5 65) (end 115.225 64.275) (width 0.2) (layer "F.Cu") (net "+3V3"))
 (segment (start 102.85 55.525) (end 102.675 55.35) (width 0.2) (layer "F.Cu") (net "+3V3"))
 (segment (start 105 59) (end 106.5 60.5) (width 0.2) (layer "F.Cu") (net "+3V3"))
 (segment (start 103.325 57.025) (end 103.325 56.575) (width 0.2) (layer "F.Cu") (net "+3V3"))
 (segment (start 115.225 64.275) (end 115.225 62.5) (width 0.2) (layer "F.Cu") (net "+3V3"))
 (segment (start 98.5 59) (end 100.475 57.025) (width 0.2) (layer "F.Cu") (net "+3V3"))
 (segment (start 112 52.869328) (end 112 60.5) (width 0.2) (layer "F.Cu") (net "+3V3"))
 (segment (start 116.6 58.550001) (end 117.100001 58.05) (width 0.2) (layer "F.Cu") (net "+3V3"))
 (segment (start 112 60.5) (end 113 61.5) (width 0.2) (layer "F.Cu") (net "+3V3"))
 (segment (start 114.919328 49.95) (end 112 52.869328) (width 0.2) (layer "F.Cu") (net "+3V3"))
 (segment (start 102.675 55.35) (end 102.675 54.975) (width 0.2) (layer "F.Cu") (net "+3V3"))
 (segment (start 113 64) (end 107.5 64) (width 0.2) (layer "F.Cu") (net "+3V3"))
 (segment (start 120.55 58.05) (end 120.55 52.7) (width 0.2) (layer "F.Cu") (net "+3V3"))
 (segment (start 103.325 56.575) (end 103.425 56.475) (width 0.2) (layer "F.Cu") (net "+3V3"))
 (segment (start 116.6 51.630672) (end 116.6 51.2) (width 0.2) (layer "F.Cu") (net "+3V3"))
 (segment (start 112.45 59.015686) (end 112.45 52.419328) (width 0.2) (layer "F.Cu") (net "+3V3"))
 (segment (start 103.715686 56.475) (end 104.525 56.475) (width 0.2) (layer "F.Cu") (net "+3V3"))
 (segment (start 110 70) (end 102 70) (width 0.2) (layer "F.Cu") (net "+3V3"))
 (segment (start 100.225 60.5) (end 100.225 55.75) (width 0.2) (layer "F.Cu") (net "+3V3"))
 (segment (start 106.5 60.5) (end 106.5 64) (width 0.2) (layer "F.Cu") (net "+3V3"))
 (segment (start 100.225 55.75) (end 101.55 54.425) (width 0.2) (layer "F.Cu") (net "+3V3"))
 (segment (start 117.419328 52.45) (end 116.6 51.630672) (width 0.2) (layer "F.Cu") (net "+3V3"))
 (segment (start 116.830672 49.95) (end 116.830672 51.861344) (width 0.2) (layer "F.Cu") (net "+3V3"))
 (segment (start 100.475 57.025) (end 102.025 57.025) (width 0.2) (layer "F.Cu") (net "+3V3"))
 (segment (start 107.5 59) (end 104.025 55.525) (width 0.2) (layer "F.Cu") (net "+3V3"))
 (segment (start 115.225 62.5) (end 115.225 61.790686) (width 0.2) (layer "F.Cu") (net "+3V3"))
 (segment (start 117.619328 52.65) (end 120.55 52.65) (width 0.2) (layer "F.Cu") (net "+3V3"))
 (segment (start 120.3 52.45) (end 117.419328 52.45) (width 0.2) (layer "F.Cu") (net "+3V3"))
 (segment (start 115.780672 49.95) (end 114.919328 49.95) (width 0.2) (layer "F.Cu") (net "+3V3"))
 (segment (start 117.100001 58.05) (end 120.55 58.05) (width 0.2) (layer "F.Cu") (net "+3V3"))
 (segment (start 100.225 59) (end 100.225 60.5) (width 0.2) (layer "F.Cu") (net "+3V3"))
 (segment (start 120.55 52.65) (end 120.55 58.2) (width 0.2) (layer "F.Cu") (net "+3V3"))
 (segment (start 116.6 50.769328) (end 115.780672 49.95) (width 0.2) (layer "F.Cu") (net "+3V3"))
 (segment (start 101.55 54.425) (end 101.55 56.55) (width 0.2) (layer "F.Cu") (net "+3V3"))
 (segment (start 102.5 54.425) (end 102.5 55.259314) (width 0.2) (layer "F.Cu") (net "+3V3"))
 (segment (start 102.5 54.425) (end 101.55 54.425) (width 0.2) (layer "F.Cu") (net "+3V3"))
 (segment (start 102.675 54.975) (end 102.675 54.6) (width 0.2) (layer "F.Cu") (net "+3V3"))
 (segment (start 112.45 52.419328) (end 114.919328 49.95) (width 0.2) (layer "F.Cu") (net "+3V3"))
 (segment (start 101.315 71.315) (end 98 68) (width 0.2) (layer "F.Cu") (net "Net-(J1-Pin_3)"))
 (segment (start 115.08 70) (end 113.765 71.315) (width 0.2) (layer "F.Cu") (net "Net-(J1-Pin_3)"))
 (segment (start 122.030672 59.5) (end 123.25 58.280672) (width 0.2) (layer "F.Cu") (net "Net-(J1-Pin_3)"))
 (segment (start 123.25 58.280672) (end 123.25 52.419328) (width 0.2) (layer "F.Cu") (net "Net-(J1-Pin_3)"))
 (segment (start 108.3 49.55) (end 103.325 54.525) (width 0.2) (layer "F.Cu") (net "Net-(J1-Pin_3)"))
 (segment (start 98 68) (end 98 54) (width 0.2) (layer "F.Cu") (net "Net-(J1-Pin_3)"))
 (segment (start 124 48.5) (end 124.5 49) (width 0.2) (layer "F.Cu") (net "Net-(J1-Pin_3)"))
 (segment (start 120.35 65.35) (end 120.35 59.5) (width 0.2) (layer "F.Cu") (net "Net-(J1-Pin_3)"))
 (segment (start 113.765 71.315) (end 101.315 71.315) (width 0.2) (layer "F.Cu") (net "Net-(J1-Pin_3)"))
 (segment (start 103.5 48.5) (end 124 48.5) (width 0.2) (layer "F.Cu") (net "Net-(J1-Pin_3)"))
 (segment (start 98 54) (end 103.5 48.5) (width 0.2) (layer "F.Cu") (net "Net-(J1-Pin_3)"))
 (segment (start 124.5 49) (end 124.5 64.75) (width 0.2) (layer "F.Cu") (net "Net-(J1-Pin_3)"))
 (segment (start 123.25 52.419328) (end 120.380672 49.55) (width 0.2) (layer "F.Cu") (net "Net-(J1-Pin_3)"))
 (segment (start 124.5 64.75) (end 123.25 66) (width 0.2) (layer "F.Cu") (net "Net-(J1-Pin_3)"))
 (segment (start 123.25 66) (end 121 66) (width 0.2) (layer "F.Cu") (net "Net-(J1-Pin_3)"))
 (segment (start 120.35 59.5) (end 122.030672 59.5) (width 0.2) (layer "F.Cu") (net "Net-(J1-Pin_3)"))
 (segment (start 120.5 59.5) (end 120.35 59.5) (width 0.2) (layer "F.Cu") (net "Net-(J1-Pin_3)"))
 (segment (start 121 66) (end 120.35 65.35) (width 0.2) (layer "F.Cu") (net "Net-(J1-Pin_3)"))
 (segment (start 103.325 54.525) (end 103.325 54.975) (width 0.2) (layer "F.Cu") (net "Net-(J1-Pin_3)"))
 (segment (start 120.380672 49.55) (end 108.3 49.55) (width 0.2) (layer "F.Cu") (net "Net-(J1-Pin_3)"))
 (segment (start 101.149314 71.715) (end 97.6 68.165685) (width 0.2) (layer "F.Cu") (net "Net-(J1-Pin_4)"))
 (segment (start 97.6 68.165685) (end 97.6 53.834314) (width 0.2) (layer "F.Cu") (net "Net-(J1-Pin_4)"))
 (segment (start 117.62 70) (end 119.1 68.52) (width 0.2) (layer "F.Cu") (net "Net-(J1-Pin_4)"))
 (segment (start 97.6 53.834314) (end 101.075735 50.358579) (width 0.2) (layer "F.Cu") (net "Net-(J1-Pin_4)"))
 (segment (start 119.1 68.52) (end 119.1 59.5) (width 0.2) (layer "F.Cu") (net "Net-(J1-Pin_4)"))
 (segment (start 115.905 71.715) (end 101.149314 71.715) (width 0.2) (layer "F.Cu") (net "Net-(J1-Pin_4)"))
 (segment (start 106 54) (end 105.025 54.975) (width 0.2) (layer "F.Cu") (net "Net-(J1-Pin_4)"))
 (segment (start 101.075735 50.358579) (end 101.075735 50.075735) (width 0.2) (layer "F.Cu") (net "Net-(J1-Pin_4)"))
 (segment (start 117.62 70) (end 115.905 71.715) (width 0.2) (layer "F.Cu") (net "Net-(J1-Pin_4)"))
 (segment (start 105.025 54.975) (end 103.975 54.975) (width 0.2) (layer "F.Cu") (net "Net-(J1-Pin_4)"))
 (via (at 106 54) (size 0.6) (drill 0.3) (layers "F.Cu" "B.Cu") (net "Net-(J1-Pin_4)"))
 (via (at 101.075735 50.075735) (size 0.6) (drill 0.3) (layers "F.Cu" "B.Cu") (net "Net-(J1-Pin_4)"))
 (segment (start 105 54) (end 106 54) (width 0.2) (layer "B.Cu") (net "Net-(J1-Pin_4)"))
 (segment (start 101.075735 50.075735) (end 105 54) (width 0.2) (layer "B.Cu") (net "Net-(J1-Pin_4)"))
 (segment (start 103.975 62.2) (end 103.675 62.5) (width 0.2) (layer "F.Cu") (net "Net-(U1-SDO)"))
 (segment (start 103.975 57.025) (end 103.975 62.2) (width 0.2) (layer "F.Cu") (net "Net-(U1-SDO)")))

